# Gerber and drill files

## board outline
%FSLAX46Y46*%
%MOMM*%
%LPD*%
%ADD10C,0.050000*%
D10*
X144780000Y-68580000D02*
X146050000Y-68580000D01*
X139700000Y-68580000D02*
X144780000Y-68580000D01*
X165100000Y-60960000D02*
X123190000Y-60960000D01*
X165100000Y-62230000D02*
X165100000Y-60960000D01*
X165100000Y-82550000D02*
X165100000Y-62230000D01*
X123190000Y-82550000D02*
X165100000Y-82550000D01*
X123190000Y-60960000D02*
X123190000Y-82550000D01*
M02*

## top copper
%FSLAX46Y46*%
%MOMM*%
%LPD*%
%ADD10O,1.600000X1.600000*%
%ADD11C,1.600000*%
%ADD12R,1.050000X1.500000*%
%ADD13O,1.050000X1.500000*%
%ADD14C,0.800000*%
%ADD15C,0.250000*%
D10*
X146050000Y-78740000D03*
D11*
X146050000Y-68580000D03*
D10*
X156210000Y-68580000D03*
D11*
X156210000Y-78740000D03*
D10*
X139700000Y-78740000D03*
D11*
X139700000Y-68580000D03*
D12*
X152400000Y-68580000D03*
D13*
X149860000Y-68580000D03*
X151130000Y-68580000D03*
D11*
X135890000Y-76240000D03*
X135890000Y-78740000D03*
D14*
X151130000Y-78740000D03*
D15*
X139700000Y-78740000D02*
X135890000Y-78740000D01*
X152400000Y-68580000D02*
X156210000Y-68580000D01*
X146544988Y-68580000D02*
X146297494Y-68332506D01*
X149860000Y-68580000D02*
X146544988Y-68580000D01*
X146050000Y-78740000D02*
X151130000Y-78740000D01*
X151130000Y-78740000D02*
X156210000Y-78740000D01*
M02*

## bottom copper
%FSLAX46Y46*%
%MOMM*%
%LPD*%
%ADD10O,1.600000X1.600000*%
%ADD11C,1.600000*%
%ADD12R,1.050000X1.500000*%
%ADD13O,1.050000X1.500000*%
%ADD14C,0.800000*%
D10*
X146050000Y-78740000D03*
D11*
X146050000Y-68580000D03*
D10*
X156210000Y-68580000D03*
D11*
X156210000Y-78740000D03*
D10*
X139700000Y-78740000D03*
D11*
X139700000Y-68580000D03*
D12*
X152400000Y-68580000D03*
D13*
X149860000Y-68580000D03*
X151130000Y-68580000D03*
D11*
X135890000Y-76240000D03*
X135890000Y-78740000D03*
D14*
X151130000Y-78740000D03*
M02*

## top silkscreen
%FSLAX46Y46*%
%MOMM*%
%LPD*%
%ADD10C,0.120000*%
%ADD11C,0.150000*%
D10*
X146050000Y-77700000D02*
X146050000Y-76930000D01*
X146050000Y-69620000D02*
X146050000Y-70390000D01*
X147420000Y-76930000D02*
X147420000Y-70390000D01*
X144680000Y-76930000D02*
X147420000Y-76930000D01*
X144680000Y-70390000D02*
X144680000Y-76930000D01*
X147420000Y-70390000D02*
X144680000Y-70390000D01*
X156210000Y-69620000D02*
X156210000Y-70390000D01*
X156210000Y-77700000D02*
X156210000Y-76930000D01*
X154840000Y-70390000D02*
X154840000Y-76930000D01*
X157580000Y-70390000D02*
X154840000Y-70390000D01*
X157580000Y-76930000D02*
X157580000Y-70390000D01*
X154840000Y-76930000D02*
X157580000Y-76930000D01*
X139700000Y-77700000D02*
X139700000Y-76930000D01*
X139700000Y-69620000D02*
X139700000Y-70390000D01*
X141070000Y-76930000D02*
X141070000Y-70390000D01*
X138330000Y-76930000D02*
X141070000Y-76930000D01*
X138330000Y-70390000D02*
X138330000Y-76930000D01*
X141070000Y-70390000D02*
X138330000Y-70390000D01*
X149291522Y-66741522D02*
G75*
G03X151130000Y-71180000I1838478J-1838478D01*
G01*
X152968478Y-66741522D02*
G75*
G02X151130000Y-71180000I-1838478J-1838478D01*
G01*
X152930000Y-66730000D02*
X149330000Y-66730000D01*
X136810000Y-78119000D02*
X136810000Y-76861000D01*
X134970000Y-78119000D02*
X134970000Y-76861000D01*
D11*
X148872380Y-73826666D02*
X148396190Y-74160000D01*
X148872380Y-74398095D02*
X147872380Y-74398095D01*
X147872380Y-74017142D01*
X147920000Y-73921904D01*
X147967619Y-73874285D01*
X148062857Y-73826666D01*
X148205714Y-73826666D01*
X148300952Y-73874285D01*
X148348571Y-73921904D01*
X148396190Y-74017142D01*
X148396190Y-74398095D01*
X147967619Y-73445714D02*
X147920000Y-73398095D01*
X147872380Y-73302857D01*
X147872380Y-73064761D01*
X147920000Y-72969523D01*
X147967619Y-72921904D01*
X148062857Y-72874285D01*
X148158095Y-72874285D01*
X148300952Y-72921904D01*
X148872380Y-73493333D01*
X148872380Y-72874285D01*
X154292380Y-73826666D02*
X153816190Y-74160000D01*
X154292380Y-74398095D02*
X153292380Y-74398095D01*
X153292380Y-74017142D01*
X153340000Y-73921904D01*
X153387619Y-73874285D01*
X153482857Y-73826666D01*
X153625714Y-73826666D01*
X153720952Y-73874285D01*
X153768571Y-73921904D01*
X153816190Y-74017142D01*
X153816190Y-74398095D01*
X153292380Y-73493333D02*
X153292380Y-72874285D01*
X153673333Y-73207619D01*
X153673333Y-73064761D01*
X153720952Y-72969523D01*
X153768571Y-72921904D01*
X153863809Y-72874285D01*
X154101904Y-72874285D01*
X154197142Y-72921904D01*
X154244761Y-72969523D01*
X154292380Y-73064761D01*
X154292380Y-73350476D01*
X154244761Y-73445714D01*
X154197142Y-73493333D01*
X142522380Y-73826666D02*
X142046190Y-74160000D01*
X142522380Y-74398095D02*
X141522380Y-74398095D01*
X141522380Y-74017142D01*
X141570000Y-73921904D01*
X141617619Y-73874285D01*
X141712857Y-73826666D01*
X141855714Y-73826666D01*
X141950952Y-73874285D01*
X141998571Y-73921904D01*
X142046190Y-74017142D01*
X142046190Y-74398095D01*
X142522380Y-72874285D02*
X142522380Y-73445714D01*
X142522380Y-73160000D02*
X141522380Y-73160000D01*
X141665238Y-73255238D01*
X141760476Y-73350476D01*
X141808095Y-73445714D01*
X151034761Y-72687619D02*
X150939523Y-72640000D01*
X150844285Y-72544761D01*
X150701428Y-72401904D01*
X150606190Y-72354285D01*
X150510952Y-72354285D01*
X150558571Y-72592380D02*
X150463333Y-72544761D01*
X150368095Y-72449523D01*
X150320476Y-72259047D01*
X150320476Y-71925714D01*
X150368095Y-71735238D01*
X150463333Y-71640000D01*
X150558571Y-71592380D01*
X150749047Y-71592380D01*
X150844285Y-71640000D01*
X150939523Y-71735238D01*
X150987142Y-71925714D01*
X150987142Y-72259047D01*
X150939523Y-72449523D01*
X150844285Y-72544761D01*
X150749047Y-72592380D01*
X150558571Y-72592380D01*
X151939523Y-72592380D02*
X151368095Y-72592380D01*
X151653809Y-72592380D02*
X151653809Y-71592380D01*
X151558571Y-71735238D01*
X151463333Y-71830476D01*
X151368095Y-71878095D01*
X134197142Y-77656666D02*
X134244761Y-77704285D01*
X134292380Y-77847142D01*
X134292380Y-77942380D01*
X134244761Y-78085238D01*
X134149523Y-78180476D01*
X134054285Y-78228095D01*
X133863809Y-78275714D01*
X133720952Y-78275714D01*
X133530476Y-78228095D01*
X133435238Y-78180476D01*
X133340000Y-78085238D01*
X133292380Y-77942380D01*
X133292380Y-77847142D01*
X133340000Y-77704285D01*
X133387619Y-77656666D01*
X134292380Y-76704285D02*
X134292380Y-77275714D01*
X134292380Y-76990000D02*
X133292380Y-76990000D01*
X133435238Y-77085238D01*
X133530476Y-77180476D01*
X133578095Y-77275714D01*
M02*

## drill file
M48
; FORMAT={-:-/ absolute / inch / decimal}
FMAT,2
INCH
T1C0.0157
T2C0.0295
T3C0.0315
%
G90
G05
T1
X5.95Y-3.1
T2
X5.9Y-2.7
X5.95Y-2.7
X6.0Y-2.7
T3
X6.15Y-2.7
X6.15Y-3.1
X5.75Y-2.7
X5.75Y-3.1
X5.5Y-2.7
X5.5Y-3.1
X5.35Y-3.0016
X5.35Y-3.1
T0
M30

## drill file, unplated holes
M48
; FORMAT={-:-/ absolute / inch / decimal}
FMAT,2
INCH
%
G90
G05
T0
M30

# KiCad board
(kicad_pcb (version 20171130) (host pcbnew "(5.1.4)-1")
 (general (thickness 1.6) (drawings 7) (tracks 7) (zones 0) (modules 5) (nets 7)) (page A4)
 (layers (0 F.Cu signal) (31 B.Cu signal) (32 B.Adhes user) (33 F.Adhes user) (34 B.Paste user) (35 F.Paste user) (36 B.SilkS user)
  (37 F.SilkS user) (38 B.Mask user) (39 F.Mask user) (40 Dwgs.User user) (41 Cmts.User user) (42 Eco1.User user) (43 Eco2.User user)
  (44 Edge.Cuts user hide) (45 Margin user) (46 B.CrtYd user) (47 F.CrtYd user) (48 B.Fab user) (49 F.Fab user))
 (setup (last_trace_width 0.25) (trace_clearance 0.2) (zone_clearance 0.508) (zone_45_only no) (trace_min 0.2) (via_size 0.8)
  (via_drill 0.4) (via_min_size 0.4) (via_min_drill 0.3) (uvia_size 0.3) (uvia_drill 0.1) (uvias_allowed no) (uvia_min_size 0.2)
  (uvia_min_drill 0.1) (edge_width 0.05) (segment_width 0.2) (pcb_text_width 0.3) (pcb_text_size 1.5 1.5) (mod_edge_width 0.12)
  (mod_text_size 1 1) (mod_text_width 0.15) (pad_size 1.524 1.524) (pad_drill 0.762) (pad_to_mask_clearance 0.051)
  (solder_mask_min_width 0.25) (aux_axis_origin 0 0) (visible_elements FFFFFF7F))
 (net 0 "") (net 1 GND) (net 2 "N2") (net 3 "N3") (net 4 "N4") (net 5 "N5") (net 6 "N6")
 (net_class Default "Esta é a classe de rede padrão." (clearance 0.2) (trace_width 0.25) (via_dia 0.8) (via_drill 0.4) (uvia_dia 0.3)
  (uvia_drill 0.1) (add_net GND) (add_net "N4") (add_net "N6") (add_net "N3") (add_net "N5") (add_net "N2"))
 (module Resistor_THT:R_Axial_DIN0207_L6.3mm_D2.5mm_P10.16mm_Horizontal (layer F.Cu) (at 146.05 68.58 270)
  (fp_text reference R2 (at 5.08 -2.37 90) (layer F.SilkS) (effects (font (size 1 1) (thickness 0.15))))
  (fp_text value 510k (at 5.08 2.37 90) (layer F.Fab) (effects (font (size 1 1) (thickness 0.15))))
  (fp_line (start 9.12 0) (end 8.35 0) (layer F.SilkS) (width 0.12))
  (fp_line (start 1.04 0) (end 1.81 0) (layer F.SilkS) (width 0.12))
  (fp_line (start 8.35 -1.37) (end 1.81 -1.37) (layer F.SilkS) (width 0.12))
  (fp_line (start 8.35 1.37) (end 8.35 -1.37) (layer F.SilkS) (width 0.12))
  (fp_line (start 1.81 1.37) (end 8.35 1.37) (layer F.SilkS) (width 0.12))
  (fp_line (start 1.81 -1.37) (end 1.81 1.37) (layer F.SilkS) (width 0.12))
  (pad 2 thru_hole oval (at 10.16 0 270) (size 1.6 1.6) (drill 0.8) (layers *.Cu *.Mask) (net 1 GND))
  (pad 1 thru_hole circle (at 0 0 270) (size 1.6 1.6) (drill 0.8) (layers *.Cu *.Mask) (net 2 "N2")))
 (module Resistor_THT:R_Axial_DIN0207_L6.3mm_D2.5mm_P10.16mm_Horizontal (layer F.Cu) (at 156.21 78.74 90)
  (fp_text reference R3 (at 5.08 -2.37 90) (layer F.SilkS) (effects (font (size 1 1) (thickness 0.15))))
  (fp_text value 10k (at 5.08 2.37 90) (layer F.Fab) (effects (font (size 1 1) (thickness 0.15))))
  (fp_line (start 9.12 0) (end 8.35 0) (layer F.SilkS) (width 0.12))
  (fp_line (start 1.04 0) (end 1.81 0) (layer F.SilkS) (width 0.12))
  (fp_line (start 8.35 -1.37) (end 1.81 -1.37) (layer F.SilkS) (width 0.12))
  (fp_line (start 8.35 1.37) (end 8.35 -1.37) (layer F.SilkS) (width 0.12))
  (fp_line (start 1.81 1.37) (end 8.35 1.37) (layer F.SilkS) (width 0.12))
  (fp_line (start 1.81 -1.37) (end 1.81 1.37) (layer F.SilkS) (width 0.12))
  (pad 2 thru_hole oval (at 10.16 0 90) (size 1.6 1.6) (drill 0.8) (layers *.Cu *.Mask) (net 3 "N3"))
  (pad 1 thru_hole circle (at 0 0 90) (size 1.6 1.6) (drill 0.8) (layers *.Cu *.Mask) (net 1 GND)))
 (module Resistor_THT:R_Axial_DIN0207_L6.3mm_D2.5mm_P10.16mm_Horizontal (layer F.Cu) (at 139.7 68.58 270)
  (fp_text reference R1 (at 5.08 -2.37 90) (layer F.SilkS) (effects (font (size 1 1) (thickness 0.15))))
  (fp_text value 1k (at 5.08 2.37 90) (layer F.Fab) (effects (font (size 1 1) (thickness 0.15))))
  (fp_line (start 9.12 0) (end 8.35 0) (layer F.SilkS) (width 0.12))
  (fp_line (start 1.04 0) (end 1.81 0) (layer F.SilkS) (width 0.12))
  (fp_line (start 8.35 -1.37) (end 1.81 -1.37) (layer F.SilkS) (width 0.12))
  (fp_line (start 8.35 1.37) (end 8.35 -1.37) (layer F.SilkS) (width 0.12))
  (fp_line (start 1.81 1.37) (end 8.35 1.37) (layer F.SilkS) (width 0.12))
  (fp_line (start 1.81 -1.37) (end 1.81 1.37) (layer F.SilkS) (width 0.12))
  (pad 2 thru_hole oval (at 10.16 0 270) (size 1.6 1.6) (drill 0.8) (layers *.Cu *.Mask) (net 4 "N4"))
  (pad 1 thru_hole circle (at 0 0 270) (size 1.6 1.6) (drill 0.8) (layers *.Cu *.Mask) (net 2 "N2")))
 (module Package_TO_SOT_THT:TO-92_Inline (layer F.Cu) (at 152.4 68.58 180)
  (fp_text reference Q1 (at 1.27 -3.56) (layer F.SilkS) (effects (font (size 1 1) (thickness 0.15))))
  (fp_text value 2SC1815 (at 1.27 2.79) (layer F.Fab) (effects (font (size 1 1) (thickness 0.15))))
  (fp_arc (start 1.27 0) (end 1.27 -2.6) (angle 135) (layer F.SilkS) (width 0.12))
  (fp_arc (start 1.27 0) (end 1.27 -2.6) (angle -135) (layer F.SilkS) (width 0.12))
  (fp_line (start -0.53 1.85) (end 3.07 1.85) (layer F.SilkS) (width 0.12))
  (pad 1 thru_hole rect (at 0 0 180) (size 1.05 1.5) (drill 0.75) (layers *.Cu *.Mask) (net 3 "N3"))
  (pad 3 thru_hole oval (at 2.54 0 180) (size 1.05 1.5) (drill 0.75) (layers *.Cu *.Mask) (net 2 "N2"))
  (pad 2 thru_hole oval (at 1.27 0 180) (size 1.05 1.5) (drill 0.75) (layers *.Cu *.Mask) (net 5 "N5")))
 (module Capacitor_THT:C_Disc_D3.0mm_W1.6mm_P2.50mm (layer F.Cu) (at 135.89 78.74 90)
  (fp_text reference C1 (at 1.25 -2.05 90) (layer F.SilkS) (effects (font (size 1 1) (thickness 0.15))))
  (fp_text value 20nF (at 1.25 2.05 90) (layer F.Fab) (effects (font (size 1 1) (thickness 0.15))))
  (fp_line (start 0.621 0.92) (end 1.879 0.92) (layer F.SilkS) (width 0.12))
  (fp_line (start 0.621 -0.92) (end 1.879 -0.92) (layer F.SilkS) (width 0.12))
  (pad 2 thru_hole circle (at 2.5 0 90) (size 1.6 1.6) (drill 0.8) (layers *.Cu *.Mask) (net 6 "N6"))
  (pad 1 thru_hole circle (at 0 0 90) (size 1.6 1.6) (drill 0.8) (layers *.Cu *.Mask) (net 4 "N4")))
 (gr_line (start 144.78 68.58) (end 146.05 68.58) (layer Edge.Cuts) (width 0.05))
 (gr_line (start 139.7 68.58) (end 144.78 68.58) (layer Edge.Cuts) (width 0.05))
 (gr_line (start 165.1 60.96) (end 123.19 60.96) (layer Edge.Cuts) (width 0.05))
 (gr_line (start 165.1 62.23) (end 165.1 60.96) (layer Edge.Cuts) (width 0.05))
 (gr_line (start 165.1 82.55) (end 165.1 62.23) (layer Edge.Cuts) (width 0.05))
 (gr_line (start 123.19 82.55) (end 165.1 82.55) (layer Edge.Cuts) (width 0.05))
 (gr_line (start 123.19 60.96) (end 123.19 82.55) (layer Edge.Cuts) (width 0.05))
 (segment (start 139.7 78.74) (end 135.89 78.74) (width 0.25) (layer F.Cu) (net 4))
 (segment (start 152.4 68.58) (end 156.21 68.58) (width 0.25) (layer F.Cu) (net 3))
 (segment (start 146.544988 68.58) (end 146.297494 68.332506) (width 0.25) (layer F.Cu) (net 2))
 (segment (start 149.86 68.58) (end 146.544988 68.58) (width 0.25) (layer F.Cu) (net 2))
 (via (at 151.13 78.74) (size 0.8) (drill 0.4) (layers F.Cu B.Cu) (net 1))
 (segment (start 146.05 78.74) (end 151.13 78.74) (width 0.25) (layer F.Cu) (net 1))
 (segment (start 151.13 78.74) (end 156.21 78.74) (width 0.25) (layer F.Cu) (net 1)))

